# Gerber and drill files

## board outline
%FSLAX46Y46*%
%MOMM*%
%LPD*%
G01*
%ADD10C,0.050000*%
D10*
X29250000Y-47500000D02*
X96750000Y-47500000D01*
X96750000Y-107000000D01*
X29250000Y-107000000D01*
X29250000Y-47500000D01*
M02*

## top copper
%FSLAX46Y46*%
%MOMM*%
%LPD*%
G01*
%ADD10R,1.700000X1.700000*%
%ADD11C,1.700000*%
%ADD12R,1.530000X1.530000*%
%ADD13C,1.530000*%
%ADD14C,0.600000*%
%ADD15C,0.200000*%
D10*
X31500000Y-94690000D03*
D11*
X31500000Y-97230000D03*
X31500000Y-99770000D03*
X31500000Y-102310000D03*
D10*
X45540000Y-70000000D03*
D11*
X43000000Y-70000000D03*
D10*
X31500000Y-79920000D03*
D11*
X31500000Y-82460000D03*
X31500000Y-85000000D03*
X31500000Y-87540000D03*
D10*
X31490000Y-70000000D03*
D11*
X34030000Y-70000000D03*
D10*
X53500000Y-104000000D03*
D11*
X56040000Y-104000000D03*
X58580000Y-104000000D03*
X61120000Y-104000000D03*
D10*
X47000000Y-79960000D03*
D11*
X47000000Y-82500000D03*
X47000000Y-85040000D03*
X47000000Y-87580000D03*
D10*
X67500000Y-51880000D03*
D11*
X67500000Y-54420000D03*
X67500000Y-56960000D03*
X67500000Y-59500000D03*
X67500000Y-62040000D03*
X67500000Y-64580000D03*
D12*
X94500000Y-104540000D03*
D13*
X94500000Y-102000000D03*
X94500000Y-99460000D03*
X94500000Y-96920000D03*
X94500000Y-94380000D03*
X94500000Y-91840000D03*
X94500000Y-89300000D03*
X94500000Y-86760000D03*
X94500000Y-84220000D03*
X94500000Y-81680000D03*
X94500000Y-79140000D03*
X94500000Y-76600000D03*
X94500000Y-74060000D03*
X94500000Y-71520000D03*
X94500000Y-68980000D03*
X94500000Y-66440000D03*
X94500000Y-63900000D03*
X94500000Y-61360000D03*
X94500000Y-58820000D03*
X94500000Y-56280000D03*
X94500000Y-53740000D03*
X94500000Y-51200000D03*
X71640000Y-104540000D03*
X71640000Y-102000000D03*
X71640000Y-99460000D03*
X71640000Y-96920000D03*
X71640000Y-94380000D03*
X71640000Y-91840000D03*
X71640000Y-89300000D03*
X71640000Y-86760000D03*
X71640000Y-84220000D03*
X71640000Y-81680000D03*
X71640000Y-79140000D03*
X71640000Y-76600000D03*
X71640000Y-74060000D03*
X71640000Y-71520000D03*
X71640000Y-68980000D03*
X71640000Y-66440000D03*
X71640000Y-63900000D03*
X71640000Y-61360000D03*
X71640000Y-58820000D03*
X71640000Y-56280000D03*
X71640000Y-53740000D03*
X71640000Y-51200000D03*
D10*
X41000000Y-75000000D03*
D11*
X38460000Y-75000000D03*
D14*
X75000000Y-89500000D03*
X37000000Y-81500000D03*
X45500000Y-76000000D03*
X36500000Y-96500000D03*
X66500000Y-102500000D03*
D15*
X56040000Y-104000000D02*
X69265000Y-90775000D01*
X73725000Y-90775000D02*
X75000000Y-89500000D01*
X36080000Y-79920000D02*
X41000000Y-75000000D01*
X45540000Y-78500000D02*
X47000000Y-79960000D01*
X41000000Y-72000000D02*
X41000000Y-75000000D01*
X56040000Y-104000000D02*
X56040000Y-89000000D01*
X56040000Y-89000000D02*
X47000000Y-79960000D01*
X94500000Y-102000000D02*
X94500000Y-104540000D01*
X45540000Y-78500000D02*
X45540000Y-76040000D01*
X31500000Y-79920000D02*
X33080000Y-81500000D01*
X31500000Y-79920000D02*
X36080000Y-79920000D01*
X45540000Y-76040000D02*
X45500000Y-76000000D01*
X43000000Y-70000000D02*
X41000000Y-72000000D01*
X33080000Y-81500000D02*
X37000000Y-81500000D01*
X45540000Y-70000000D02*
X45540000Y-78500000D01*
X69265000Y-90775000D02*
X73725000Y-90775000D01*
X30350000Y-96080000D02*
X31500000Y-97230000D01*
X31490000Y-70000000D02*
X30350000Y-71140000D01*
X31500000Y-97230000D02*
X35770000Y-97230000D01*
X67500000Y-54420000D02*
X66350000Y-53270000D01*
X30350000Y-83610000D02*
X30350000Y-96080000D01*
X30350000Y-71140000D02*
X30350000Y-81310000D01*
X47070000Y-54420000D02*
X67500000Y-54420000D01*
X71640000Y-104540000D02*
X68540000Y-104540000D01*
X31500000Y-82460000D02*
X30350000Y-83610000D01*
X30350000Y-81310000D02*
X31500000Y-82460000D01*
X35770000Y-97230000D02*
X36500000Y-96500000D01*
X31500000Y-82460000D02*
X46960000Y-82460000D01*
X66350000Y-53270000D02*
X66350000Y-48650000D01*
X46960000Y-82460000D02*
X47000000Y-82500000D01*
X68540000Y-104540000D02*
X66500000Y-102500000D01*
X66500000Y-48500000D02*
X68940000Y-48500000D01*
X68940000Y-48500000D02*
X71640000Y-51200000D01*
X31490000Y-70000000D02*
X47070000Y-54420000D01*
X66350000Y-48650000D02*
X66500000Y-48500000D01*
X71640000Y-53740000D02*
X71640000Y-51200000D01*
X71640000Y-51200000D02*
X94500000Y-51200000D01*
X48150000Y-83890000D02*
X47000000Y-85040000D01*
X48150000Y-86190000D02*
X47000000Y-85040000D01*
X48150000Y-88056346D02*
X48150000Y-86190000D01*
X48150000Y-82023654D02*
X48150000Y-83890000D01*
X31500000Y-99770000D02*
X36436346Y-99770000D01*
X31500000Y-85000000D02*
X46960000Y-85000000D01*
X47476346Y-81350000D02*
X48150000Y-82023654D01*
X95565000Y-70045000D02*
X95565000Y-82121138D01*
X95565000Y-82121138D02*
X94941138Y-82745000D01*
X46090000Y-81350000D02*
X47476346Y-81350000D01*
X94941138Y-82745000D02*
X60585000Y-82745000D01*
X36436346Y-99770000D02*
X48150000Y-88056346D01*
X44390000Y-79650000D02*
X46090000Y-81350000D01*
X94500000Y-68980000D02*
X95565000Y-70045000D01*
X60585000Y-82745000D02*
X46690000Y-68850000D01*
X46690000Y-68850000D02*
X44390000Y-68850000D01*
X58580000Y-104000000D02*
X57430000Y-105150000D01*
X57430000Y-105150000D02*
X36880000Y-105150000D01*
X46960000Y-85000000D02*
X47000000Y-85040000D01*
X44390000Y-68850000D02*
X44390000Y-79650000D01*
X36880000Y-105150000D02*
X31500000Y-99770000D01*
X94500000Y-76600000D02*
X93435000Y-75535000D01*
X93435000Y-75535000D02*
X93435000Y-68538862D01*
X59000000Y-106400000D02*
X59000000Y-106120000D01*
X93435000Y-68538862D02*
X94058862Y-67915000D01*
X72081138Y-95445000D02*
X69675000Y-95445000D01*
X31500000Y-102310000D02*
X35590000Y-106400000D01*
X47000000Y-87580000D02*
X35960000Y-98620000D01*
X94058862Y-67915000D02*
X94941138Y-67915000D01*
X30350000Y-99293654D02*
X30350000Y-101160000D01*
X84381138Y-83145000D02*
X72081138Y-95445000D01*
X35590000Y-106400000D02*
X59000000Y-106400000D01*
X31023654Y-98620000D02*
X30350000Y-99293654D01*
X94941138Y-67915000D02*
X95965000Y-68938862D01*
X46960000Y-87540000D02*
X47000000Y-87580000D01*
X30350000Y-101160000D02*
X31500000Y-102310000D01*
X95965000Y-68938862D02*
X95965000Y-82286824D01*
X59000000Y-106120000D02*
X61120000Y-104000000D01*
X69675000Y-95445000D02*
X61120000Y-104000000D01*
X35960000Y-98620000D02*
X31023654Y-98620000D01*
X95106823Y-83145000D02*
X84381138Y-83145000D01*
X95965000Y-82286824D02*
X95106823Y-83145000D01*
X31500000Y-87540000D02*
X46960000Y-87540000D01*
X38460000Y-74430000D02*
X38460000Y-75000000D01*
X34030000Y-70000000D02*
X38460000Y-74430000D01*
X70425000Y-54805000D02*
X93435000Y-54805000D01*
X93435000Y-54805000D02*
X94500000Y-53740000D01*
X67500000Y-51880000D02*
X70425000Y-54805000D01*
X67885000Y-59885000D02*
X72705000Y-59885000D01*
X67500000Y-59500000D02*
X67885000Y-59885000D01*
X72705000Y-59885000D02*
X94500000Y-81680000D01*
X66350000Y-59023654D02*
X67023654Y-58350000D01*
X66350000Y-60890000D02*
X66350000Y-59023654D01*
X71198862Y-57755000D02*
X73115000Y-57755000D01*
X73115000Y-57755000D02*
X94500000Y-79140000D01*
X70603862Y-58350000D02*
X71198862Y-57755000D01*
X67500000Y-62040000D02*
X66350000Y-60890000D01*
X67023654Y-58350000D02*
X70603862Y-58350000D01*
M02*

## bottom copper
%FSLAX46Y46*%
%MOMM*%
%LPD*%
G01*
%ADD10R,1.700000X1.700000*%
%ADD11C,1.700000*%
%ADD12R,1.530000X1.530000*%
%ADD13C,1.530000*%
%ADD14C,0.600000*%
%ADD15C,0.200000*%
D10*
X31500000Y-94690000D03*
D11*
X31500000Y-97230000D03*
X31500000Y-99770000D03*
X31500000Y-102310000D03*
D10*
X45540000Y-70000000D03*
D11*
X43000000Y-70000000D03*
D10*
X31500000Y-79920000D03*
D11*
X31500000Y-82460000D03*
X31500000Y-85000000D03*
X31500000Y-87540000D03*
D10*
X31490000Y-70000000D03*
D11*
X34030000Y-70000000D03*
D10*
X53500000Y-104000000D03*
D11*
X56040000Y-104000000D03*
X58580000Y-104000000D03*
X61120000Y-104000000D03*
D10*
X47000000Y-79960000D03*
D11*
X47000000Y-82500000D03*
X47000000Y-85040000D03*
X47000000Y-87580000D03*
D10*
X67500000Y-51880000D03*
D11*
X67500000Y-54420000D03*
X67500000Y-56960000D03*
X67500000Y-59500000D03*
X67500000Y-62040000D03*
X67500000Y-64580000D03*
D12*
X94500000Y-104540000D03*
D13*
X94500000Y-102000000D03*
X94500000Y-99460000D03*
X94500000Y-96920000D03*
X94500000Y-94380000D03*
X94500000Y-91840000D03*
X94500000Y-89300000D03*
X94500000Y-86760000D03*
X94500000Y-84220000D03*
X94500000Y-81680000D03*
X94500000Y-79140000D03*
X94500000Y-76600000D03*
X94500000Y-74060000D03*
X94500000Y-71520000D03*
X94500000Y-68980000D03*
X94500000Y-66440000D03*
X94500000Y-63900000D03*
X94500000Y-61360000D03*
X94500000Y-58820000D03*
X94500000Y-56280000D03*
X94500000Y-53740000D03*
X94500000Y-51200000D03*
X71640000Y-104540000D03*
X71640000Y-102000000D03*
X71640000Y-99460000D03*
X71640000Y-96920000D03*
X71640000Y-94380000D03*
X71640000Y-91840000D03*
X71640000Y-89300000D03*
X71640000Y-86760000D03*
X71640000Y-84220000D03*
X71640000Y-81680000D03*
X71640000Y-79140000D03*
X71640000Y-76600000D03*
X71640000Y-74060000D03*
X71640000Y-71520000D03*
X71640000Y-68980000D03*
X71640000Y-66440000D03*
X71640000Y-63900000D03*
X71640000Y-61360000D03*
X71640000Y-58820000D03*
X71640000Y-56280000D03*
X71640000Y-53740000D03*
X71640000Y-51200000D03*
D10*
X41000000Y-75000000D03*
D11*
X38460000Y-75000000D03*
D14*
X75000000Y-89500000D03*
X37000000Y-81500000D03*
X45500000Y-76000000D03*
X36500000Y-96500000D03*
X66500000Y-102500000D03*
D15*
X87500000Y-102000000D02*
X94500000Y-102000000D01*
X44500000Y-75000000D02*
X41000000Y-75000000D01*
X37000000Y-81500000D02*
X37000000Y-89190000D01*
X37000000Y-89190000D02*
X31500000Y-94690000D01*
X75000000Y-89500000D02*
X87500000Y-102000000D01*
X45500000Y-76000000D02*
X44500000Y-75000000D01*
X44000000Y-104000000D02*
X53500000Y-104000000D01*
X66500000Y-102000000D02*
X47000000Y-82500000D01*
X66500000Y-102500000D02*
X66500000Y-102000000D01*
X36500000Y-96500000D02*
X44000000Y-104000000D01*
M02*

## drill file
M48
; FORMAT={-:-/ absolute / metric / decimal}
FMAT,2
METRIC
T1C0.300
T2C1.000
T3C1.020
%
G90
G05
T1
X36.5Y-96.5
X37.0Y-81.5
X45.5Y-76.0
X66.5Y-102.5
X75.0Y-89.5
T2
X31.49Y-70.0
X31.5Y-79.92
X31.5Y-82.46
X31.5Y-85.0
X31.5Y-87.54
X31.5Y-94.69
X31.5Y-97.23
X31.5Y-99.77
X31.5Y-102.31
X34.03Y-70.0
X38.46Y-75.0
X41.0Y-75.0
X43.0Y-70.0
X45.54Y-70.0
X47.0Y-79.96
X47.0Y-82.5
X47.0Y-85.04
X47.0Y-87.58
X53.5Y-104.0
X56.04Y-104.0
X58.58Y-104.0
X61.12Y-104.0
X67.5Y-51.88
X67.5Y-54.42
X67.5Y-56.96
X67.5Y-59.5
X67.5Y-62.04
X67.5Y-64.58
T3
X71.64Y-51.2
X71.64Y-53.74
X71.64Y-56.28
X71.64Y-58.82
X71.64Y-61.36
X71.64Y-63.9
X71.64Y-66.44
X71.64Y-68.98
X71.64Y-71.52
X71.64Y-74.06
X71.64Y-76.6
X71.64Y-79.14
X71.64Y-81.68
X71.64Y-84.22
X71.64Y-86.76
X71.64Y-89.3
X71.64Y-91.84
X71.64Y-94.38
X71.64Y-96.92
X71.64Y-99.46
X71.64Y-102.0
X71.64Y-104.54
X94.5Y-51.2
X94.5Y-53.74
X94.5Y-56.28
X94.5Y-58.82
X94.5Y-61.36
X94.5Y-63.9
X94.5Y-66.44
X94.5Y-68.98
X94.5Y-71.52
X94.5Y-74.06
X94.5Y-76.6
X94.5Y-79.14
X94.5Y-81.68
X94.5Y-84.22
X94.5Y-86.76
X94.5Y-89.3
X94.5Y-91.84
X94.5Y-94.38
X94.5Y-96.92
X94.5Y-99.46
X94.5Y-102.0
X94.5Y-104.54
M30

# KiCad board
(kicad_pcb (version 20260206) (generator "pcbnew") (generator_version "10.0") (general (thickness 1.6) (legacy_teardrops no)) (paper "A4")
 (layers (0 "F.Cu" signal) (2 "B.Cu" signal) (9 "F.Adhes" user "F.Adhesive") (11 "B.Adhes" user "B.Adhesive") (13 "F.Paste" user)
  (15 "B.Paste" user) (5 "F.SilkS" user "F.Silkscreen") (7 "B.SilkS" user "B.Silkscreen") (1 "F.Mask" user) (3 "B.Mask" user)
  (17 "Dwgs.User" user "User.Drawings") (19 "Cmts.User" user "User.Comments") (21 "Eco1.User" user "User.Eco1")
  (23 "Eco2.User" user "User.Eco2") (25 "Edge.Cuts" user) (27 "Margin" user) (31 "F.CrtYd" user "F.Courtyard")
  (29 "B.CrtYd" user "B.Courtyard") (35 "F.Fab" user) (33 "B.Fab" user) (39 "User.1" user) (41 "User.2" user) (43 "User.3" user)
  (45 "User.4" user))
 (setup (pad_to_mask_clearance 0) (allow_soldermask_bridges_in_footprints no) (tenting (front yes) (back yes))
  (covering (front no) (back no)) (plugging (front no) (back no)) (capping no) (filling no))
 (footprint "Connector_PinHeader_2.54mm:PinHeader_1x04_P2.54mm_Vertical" (layer "F.Cu") (at 31.5 94.69)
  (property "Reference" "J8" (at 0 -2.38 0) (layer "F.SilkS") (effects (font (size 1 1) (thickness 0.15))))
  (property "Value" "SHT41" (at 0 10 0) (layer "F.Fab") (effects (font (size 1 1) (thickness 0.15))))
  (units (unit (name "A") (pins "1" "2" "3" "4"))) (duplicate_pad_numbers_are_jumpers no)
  (pad "1" thru_hole rect (at 0 0) (size 1.7 1.7) (drill 1) (layers "*.Cu" "*.Mask") (remove_unused_layers no) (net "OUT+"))
  (pad "2" thru_hole circle (at 0 2.54) (size 1.7 1.7) (drill 1) (layers "*.Cu" "*.Mask") (remove_unused_layers no) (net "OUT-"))
  (pad "3" thru_hole circle (at 0 5.08) (size 1.7 1.7) (drill 1) (layers "*.Cu" "*.Mask") (remove_unused_layers no) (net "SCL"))
  (pad "4" thru_hole circle (at 0 7.62) (size 1.7 1.7) (drill 1) (layers "*.Cu" "*.Mask") (remove_unused_layers no) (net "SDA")))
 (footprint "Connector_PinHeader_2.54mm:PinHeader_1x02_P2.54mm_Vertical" (layer "F.Cu") (at 45.54 70 -90)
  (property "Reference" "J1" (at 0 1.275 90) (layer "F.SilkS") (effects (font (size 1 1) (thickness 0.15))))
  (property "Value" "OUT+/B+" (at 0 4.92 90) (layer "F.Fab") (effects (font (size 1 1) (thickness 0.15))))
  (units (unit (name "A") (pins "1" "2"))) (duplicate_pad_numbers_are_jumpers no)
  (pad "1" thru_hole rect (at 0 0 270) (size 1.7 1.7) (drill 1) (layers "*.Cu" "*.Mask") (remove_unused_layers no) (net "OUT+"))
  (pad "2" thru_hole circle (at 0 2.54 270) (size 1.7 1.7) (drill 1) (layers "*.Cu" "*.Mask") (remove_unused_layers no) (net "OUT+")))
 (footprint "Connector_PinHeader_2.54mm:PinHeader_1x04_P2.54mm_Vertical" (layer "F.Cu") (at 31.5 79.92)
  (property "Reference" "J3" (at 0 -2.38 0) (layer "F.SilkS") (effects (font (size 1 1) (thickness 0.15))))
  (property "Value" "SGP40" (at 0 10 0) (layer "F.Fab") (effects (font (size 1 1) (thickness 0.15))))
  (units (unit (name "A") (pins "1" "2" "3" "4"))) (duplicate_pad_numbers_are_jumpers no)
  (pad "1" thru_hole rect (at 0 0) (size 1.7 1.7) (drill 1) (layers "*.Cu" "*.Mask") (remove_unused_layers no) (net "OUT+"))
  (pad "2" thru_hole circle (at 0 2.54) (size 1.7 1.7) (drill 1) (layers "*.Cu" "*.Mask") (remove_unused_layers no) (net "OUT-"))
  (pad "3" thru_hole circle (at 0 5.08) (size 1.7 1.7) (drill 1) (layers "*.Cu" "*.Mask") (remove_unused_layers no) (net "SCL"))
  (pad "4" thru_hole circle (at 0 7.62) (size 1.7 1.7) (drill 1) (layers "*.Cu" "*.Mask") (remove_unused_layers no) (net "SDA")))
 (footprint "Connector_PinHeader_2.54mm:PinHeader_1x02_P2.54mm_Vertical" (layer "F.Cu") (at 31.49 70 90)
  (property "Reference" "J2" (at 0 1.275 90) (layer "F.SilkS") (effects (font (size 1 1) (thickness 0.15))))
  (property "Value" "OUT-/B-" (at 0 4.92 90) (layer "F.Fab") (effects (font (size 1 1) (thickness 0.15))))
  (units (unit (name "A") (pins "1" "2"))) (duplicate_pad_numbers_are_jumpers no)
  (pad "1" thru_hole rect (at 0 0 90) (size 1.7 1.7) (drill 1) (layers "*.Cu" "*.Mask") (remove_unused_layers no) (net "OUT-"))
  (pad "2" thru_hole circle (at 0 2.54 90) (size 1.7 1.7) (drill 1) (layers "*.Cu" "*.Mask") (remove_unused_layers no)
   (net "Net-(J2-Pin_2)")))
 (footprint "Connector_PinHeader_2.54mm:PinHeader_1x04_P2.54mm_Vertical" (layer "F.Cu") (at 53.5 104 90)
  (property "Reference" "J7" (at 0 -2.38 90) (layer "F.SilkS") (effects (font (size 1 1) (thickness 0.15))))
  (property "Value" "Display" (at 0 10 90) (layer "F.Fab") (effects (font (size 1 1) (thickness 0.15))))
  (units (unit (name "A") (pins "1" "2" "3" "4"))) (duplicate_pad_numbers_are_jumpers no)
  (pad "1" thru_hole rect (at 0 0 90) (size 1.7 1.7) (drill 1) (layers "*.Cu" "*.Mask") (remove_unused_layers no) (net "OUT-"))
  (pad "2" thru_hole circle (at 0 2.54 90) (size 1.7 1.7) (drill 1) (layers "*.Cu" "*.Mask") (remove_unused_layers no) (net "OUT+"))
  (pad "3" thru_hole circle (at 0 5.08 90) (size 1.7 1.7) (drill 1) (layers "*.Cu" "*.Mask") (remove_unused_layers no) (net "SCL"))
  (pad "4" thru_hole circle (at 0 7.62 90) (size 1.7 1.7) (drill 1) (layers "*.Cu" "*.Mask") (remove_unused_layers no) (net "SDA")))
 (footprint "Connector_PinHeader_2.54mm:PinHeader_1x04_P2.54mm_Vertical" (layer "F.Cu") (at 47 79.96)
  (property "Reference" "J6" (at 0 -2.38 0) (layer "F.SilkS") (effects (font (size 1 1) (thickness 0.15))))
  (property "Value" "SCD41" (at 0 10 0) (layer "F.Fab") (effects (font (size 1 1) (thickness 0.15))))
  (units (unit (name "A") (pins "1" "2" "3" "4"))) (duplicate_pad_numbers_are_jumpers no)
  (pad "1" thru_hole rect (at 0 0) (size 1.7 1.7) (drill 1) (layers "*.Cu" "*.Mask") (remove_unused_layers no) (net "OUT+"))
  (pad "2" thru_hole circle (at 0 2.54) (size 1.7 1.7) (drill 1) (layers "*.Cu" "*.Mask") (remove_unused_layers no) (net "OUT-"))
  (pad "3" thru_hole circle (at 0 5.08) (size 1.7 1.7) (drill 1) (layers "*.Cu" "*.Mask") (remove_unused_layers no) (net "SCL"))
  (pad "4" thru_hole circle (at 0 7.62) (size 1.7 1.7) (drill 1) (layers "*.Cu" "*.Mask") (remove_unused_layers no) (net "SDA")))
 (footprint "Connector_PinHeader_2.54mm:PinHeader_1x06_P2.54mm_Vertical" (layer "F.Cu") (at 67.5 51.88)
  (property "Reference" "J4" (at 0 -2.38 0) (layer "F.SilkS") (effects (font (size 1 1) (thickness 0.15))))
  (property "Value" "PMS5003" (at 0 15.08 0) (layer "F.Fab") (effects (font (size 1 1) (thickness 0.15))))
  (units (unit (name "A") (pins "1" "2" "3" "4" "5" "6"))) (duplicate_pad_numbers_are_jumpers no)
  (pad "1" thru_hole rect (at 0 0) (size 1.7 1.7) (drill 1) (layers "*.Cu" "*.Mask") (remove_unused_layers no) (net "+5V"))
  (pad "2" thru_hole circle (at 0 2.54) (size 1.7 1.7) (drill 1) (layers "*.Cu" "*.Mask") (remove_unused_layers no) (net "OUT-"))
  (pad "3" thru_hole circle (at 0 5.08) (size 1.7 1.7) (drill 1) (layers "*.Cu" "*.Mask") (remove_unused_layers no)
   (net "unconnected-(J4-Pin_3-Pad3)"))
  (pad "4" thru_hole circle (at 0 7.62) (size 1.7 1.7) (drill 1) (layers "*.Cu" "*.Mask") (remove_unused_layers no) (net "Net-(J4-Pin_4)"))
  (pad "5" thru_hole circle (at 0 10.16) (size 1.7 1.7) (drill 1) (layers "*.Cu" "*.Mask") (remove_unused_layers no) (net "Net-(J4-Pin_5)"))
  (pad "6" thru_hole circle (at 0 12.7) (size 1.7 1.7) (drill 1) (layers "*.Cu" "*.Mask") (remove_unused_layers no)
   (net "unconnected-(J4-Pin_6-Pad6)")))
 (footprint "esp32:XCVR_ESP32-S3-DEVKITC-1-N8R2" (layer "F.Cu") (at 83.07 74.57 180)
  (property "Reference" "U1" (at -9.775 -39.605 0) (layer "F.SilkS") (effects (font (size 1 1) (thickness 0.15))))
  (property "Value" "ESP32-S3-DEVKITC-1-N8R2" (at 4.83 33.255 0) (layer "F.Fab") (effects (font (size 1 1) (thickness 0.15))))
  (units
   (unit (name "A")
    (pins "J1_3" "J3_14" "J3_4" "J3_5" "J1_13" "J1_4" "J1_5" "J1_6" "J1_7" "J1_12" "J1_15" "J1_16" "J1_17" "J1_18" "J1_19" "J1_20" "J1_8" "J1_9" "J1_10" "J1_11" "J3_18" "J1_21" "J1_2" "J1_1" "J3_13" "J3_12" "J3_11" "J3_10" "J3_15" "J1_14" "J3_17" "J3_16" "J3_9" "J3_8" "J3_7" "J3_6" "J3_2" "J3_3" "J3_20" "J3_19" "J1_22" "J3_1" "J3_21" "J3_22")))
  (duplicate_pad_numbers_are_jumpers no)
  (pad "J1_1" thru_hole rect (at -11.43 -29.97 180) (size 1.53 1.53) (drill 1.02) (layers "*.Cu" "*.Mask") (remove_unused_layers no)
   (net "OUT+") (solder_mask_margin 0.102))
  (pad "J1_2" thru_hole circle (at -11.43 -27.43 180) (size 1.53 1.53) (drill 1.02) (layers "*.Cu" "*.Mask") (remove_unused_layers no)
   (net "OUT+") (solder_mask_margin 0.102))
  (pad "J1_3" thru_hole circle (at -11.43 -24.89 180) (size 1.53 1.53) (drill 1.02) (layers "*.Cu" "*.Mask") (remove_unused_layers no)
   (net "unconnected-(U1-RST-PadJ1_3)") (solder_mask_margin 0.102))
  (pad "J1_4" thru_hole circle (at -11.43 -22.35 180) (size 1.53 1.53) (drill 1.02) (layers "*.Cu" "*.Mask") (remove_unused_layers no)
   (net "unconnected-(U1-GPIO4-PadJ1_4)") (solder_mask_margin 0.102))
  (pad "J1_5" thru_hole circle (at -11.43 -19.81 180) (size 1.53 1.53) (drill 1.02) (layers "*.Cu" "*.Mask") (remove_unused_layers no)
   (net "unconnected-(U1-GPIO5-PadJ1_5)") (solder_mask_margin 0.102))
  (pad "J1_6" thru_hole circle (at -11.43 -17.27 180) (size 1.53 1.53) (drill 1.02) (layers "*.Cu" "*.Mask") (remove_unused_layers no)
   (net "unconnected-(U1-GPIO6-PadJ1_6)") (solder_mask_margin 0.102))
  (pad "J1_7" thru_hole circle (at -11.43 -14.73 180) (size 1.53 1.53) (drill 1.02) (layers "*.Cu" "*.Mask") (remove_unused_layers no)
   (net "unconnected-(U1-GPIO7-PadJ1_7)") (solder_mask_margin 0.102))
  (pad "J1_8" thru_hole circle (at -11.43 -12.19 180) (size 1.53 1.53) (drill 1.02) (layers "*.Cu" "*.Mask") (remove_unused_layers no)
   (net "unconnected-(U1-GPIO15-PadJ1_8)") (solder_mask_margin 0.102))
  (pad "J1_9" thru_hole circle (at -11.43 -9.65 180) (size 1.53 1.53) (drill 1.02) (layers "*.Cu" "*.Mask") (remove_unused_layers no)
   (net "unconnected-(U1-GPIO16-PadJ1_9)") (solder_mask_margin 0.102))
  (pad "J1_10" thru_hole circle (at -11.43 -7.11 180) (size 1.53 1.53) (drill 1.02) (layers "*.Cu" "*.Mask") (remove_unused_layers no)
   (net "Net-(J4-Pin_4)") (solder_mask_margin 0.102))
  (pad "J1_11" thru_hole circle (at -11.43 -4.57 180) (size 1.53 1.53) (drill 1.02) (layers "*.Cu" "*.Mask") (remove_unused_layers no)
   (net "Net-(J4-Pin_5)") (solder_mask_margin 0.102))
  (pad "J1_12" thru_hole circle (at -11.43 -2.03 180) (size 1.53 1.53) (drill 1.02) (layers "*.Cu" "*.Mask") (remove_unused_layers no)
   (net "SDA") (solder_mask_margin 0.102))
  (pad "J1_13" thru_hole circle (at -11.43 0.51 180) (size 1.53 1.53) (drill 1.02) (layers "*.Cu" "*.Mask") (remove_unused_layers no)
   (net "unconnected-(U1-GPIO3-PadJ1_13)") (solder_mask_margin 0.102))
  (pad "J1_14" thru_hole circle (at -11.43 3.05 180) (size 1.53 1.53) (drill 1.02) (layers "*.Cu" "*.Mask") (remove_unused_layers no)
   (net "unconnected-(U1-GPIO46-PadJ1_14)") (solder_mask_margin 0.102))
  (pad "J1_15" thru_hole circle (at -11.43 5.59 180) (size 1.53 1.53) (drill 1.02) (layers "*.Cu" "*.Mask") (remove_unused_layers no)
   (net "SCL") (solder_mask_margin 0.102))
  (pad "J1_16" thru_hole circle (at -11.43 8.13 180) (size 1.53 1.53) (drill 1.02) (layers "*.Cu" "*.Mask") (remove_unused_layers no)
   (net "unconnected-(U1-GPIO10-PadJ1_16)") (solder_mask_margin 0.102))
  (pad "J1_17" thru_hole circle (at -11.43 10.67 180) (size 1.53 1.53) (drill 1.02) (layers "*.Cu" "*.Mask") (remove_unused_layers no)
   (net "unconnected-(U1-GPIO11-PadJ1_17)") (solder_mask_margin 0.102))
  (pad "J1_18" thru_hole circle (at -11.43 13.21 180) (size 1.53 1.53) (drill 1.02) (layers "*.Cu" "*.Mask") (remove_unused_layers no)
   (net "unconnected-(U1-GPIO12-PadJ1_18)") (solder_mask_margin 0.102))
  (pad "J1_19" thru_hole circle (at -11.43 15.75 180) (size 1.53 1.53) (drill 1.02) (layers "*.Cu" "*.Mask") (remove_unused_layers no)
   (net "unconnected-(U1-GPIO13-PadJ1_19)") (solder_mask_margin 0.102))
  (pad "J1_20" thru_hole circle (at -11.43 18.29 180) (size 1.53 1.53) (drill 1.02) (layers "*.Cu" "*.Mask") (remove_unused_layers no)
   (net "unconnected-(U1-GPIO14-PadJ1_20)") (solder_mask_margin 0.102))
  (pad "J1_21" thru_hole circle (at -11.43 20.83 180) (size 1.53 1.53) (drill 1.02) (layers "*.Cu" "*.Mask") (remove_unused_layers no)
   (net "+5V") (solder_mask_margin 0.102))
  (pad "J1_22" thru_hole circle (at -11.43 23.37 180) (size 1.53 1.53) (drill 1.02) (layers "*.Cu" "*.Mask") (remove_unused_layers no)
   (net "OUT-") (solder_mask_margin 0.102))
  (pad "J3_1" thru_hole circle (at 11.43 -29.97 180) (size 1.53 1.53) (drill 1.02) (layers "*.Cu" "*.Mask") (remove_unused_layers no)
   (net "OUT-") (solder_mask_margin 0.102))
  (pad "J3_2" thru_hole circle (at 11.43 -27.43 180) (size 1.53 1.53) (drill 1.02) (layers "*.Cu" "*.Mask") (remove_unused_layers no)
   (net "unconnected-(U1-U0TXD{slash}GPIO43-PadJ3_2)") (solder_mask_margin 0.102))
  (pad "J3_3" thru_hole circle (at 11.43 -24.89 180) (size 1.53 1.53) (drill 1.02) (layers "*.Cu" "*.Mask") (remove_unused_layers no)
   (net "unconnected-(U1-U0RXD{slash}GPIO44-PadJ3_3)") (solder_mask_margin 0.102))
  (pad "J3_4" thru_hole circle (at 11.43 -22.35 180) (size 1.53 1.53) (drill 1.02) (layers "*.Cu" "*.Mask") (remove_unused_layers no)
   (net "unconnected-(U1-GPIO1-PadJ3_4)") (solder_mask_margin 0.102))
  (pad "J3_5" thru_hole circle (at 11.43 -19.81 180) (size 1.53 1.53) (drill 1.02) (layers "*.Cu" "*.Mask") (remove_unused_layers no)
   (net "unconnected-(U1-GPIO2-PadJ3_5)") (solder_mask_margin 0.102))
  (pad "J3_6" thru_hole circle (at 11.43 -17.27 180) (size 1.53 1.53) (drill 1.02) (layers "*.Cu" "*.Mask") (remove_unused_layers no)
   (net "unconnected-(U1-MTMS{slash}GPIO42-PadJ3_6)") (solder_mask_margin 0.102))
  (pad "J3_7" thru_hole circle (at 11.43 -14.73 180) (size 1.53 1.53) (drill 1.02) (layers "*.Cu" "*.Mask") (remove_unused_layers no)
   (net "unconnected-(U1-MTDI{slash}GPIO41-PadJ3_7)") (solder_mask_margin 0.102))
  (pad "J3_8" thru_hole circle (at 11.43 -12.19 180) (size 1.53 1.53) (drill 1.02) (layers "*.Cu" "*.Mask") (remove_unused_layers no)
   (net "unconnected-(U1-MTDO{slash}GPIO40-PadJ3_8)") (solder_mask_margin 0.102))
  (pad "J3_9" thru_hole circle (at 11.43 -9.65 180) (size 1.53 1.53) (drill 1.02) (layers "*.Cu" "*.Mask") (remove_unused_layers no)
   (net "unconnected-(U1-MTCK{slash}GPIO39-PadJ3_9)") (solder_mask_margin 0.102))
  (pad "J3_10" thru_hole circle (at 11.43 -7.11 180) (size 1.53 1.53) (drill 1.02) (layers "*.Cu" "*.Mask") (remove_unused_layers no)
   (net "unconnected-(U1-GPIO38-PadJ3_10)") (solder_mask_margin 0.102))
  (pad "J3_11" thru_hole circle (at 11.43 -4.57 180) (size 1.53 1.53) (drill 1.02) (layers "*.Cu" "*.Mask") (remove_unused_layers no)
   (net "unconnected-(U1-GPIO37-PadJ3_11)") (solder_mask_margin 0.102))
  (pad "J3_12" thru_hole circle (at 11.43 -2.03 180) (size 1.53 1.53) (drill 1.02) (layers "*.Cu" "*.Mask") (remove_unused_layers no)
   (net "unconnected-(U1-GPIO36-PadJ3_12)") (solder_mask_margin 0.102))
  (pad "J3_13" thru_hole circle (at 11.43 0.51 180) (size 1.53 1.53) (drill 1.02) (layers "*.Cu" "*.Mask") (remove_unused_layers no)
   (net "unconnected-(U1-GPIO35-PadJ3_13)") (solder_mask_margin 0.102))
  (pad "J3_14" thru_hole circle (at 11.43 3.05 180) (size 1.53 1.53) (drill 1.02) (layers "*.Cu" "*.Mask") (remove_unused_layers no)
   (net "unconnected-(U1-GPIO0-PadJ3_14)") (solder_mask_margin 0.102))
  (pad "J3_15" thru_hole circle (at 11.43 5.59 180) (size 1.53 1.53) (drill 1.02) (layers "*.Cu" "*.Mask") (remove_unused_layers no)
   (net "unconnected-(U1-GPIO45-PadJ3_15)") (solder_mask_margin 0.102))
  (pad "J3_16" thru_hole circle (at 11.43 8.13 180) (size 1.53 1.53) (drill 1.02) (layers "*.Cu" "*.Mask") (remove_unused_layers no)
   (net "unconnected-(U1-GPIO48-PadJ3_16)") (solder_mask_margin 0.102))
  (pad "J3_17" thru_hole circle (at 11.43 10.67 180) (size 1.53 1.53) (drill 1.02) (layers "*.Cu" "*.Mask") (remove_unused_layers no)
   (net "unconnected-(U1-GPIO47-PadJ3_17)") (solder_mask_margin 0.102))
  (pad "J3_18" thru_hole circle (at 11.43 13.21 180) (size 1.53 1.53) (drill 1.02) (layers "*.Cu" "*.Mask") (remove_unused_layers no)
   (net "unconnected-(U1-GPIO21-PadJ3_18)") (solder_mask_margin 0.102))
  (pad "J3_19" thru_hole circle (at 11.43 15.75 180) (size 1.53 1.53) (drill 1.02) (layers "*.Cu" "*.Mask") (remove_unused_layers no)
   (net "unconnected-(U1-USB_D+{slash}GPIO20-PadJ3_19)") (solder_mask_margin 0.102))
  (pad "J3_20" thru_hole circle (at 11.43 18.29 180) (size 1.53 1.53) (drill 1.02) (layers "*.Cu" "*.Mask") (remove_unused_layers no)
   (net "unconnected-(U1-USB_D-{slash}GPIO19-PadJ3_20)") (solder_mask_margin 0.102))
  (pad "J3_21" thru_hole circle (at 11.43 20.83 180) (size 1.53 1.53) (drill 1.02) (layers "*.Cu" "*.Mask") (remove_unused_layers no)
   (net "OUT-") (solder_mask_margin 0.102))
  (pad "J3_22" thru_hole circle (at 11.43 23.37 180) (size 1.53 1.53) (drill 1.02) (layers "*.Cu" "*.Mask") (remove_unused_layers no)
   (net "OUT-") (solder_mask_margin 0.102)))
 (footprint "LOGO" (layer "F.Cu") (at 63 98)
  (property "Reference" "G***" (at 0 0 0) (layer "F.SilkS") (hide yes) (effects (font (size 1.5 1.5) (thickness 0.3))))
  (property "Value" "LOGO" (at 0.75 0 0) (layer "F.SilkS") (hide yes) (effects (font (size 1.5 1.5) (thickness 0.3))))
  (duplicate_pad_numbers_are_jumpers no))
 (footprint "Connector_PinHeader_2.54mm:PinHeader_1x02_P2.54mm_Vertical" (layer "F.Cu") (at 41 75 -90)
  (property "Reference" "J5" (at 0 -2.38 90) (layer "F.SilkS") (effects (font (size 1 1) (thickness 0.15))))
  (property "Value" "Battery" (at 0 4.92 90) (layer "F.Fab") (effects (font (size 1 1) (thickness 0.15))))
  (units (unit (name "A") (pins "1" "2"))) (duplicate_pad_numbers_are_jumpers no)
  (pad "1" thru_hole rect (at 0 0 270) (size 1.7 1.7) (drill 1) (layers "*.Cu" "*.Mask") (remove_unused_layers no) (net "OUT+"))
  (pad "2" thru_hole circle (at 0 2.54 270) (size 1.7 1.7) (drill 1) (layers "*.Cu" "*.Mask") (remove_unused_layers no)
   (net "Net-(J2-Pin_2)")))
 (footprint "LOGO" (layer "F.Cu") (at 49.5 98)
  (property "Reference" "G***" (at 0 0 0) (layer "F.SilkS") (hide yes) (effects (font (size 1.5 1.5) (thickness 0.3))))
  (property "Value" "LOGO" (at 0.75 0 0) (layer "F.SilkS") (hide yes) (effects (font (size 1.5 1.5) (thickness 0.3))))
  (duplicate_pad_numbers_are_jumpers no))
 (gr_rect (start 29.25 47.5) (end 96.75 107) (stroke (width 0.05) (type default)) (fill no) (layer "Edge.Cuts"))
 (segment (start 56.04 104) (end 69.265 90.775) (width 0.2) (layer "F.Cu") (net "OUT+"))
 (segment (start 73.725 90.775) (end 75 89.5) (width 0.2) (layer "F.Cu") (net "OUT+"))
 (segment (start 36.08 79.92) (end 41 75) (width 0.2) (layer "F.Cu") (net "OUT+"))
 (segment (start 45.54 78.5) (end 47 79.96) (width 0.2) (layer "F.Cu") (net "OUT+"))
 (segment (start 41 72) (end 41 75) (width 0.2) (layer "F.Cu") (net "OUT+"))
 (segment (start 56.04 104) (end 56.04 89) (width 0.2) (layer "F.Cu") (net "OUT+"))
 (segment (start 56.04 89) (end 47 79.96) (width 0.2) (layer "F.Cu") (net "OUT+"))
 (segment (start 94.5 102) (end 94.5 104.54) (width 0.2) (layer "F.Cu") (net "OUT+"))
 (segment (start 45.54 78.5) (end 45.54 76.04) (width 0.2) (layer "F.Cu") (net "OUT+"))
 (segment (start 31.5 79.92) (end 33.08 81.5) (width 0.2) (layer "F.Cu") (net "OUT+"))
 (segment (start 31.5 79.92) (end 36.08 79.92) (width 0.2) (layer "F.Cu") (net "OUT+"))
 (segment (start 45.54 76.04) (end 45.5 76) (width 0.2) (layer "F.Cu") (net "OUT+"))
 (segment (start 43 70) (end 41 72) (width 0.2) (layer "F.Cu") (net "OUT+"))
 (segment (start 33.08 81.5) (end 37 81.5) (width 0.2) (layer "F.Cu") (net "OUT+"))
 (segment (start 45.54 70) (end 45.54 78.5) (width 0.2) (layer "F.Cu") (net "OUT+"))
 (segment (start 69.265 90.775) (end 73.725 90.775) (width 0.2) (layer "F.Cu") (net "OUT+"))
 (via (at 75 89.5) (size 0.6) (drill 0.3) (layers "F.Cu" "B.Cu") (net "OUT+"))
 (via (at 37 81.5) (size 0.6) (drill 0.3) (layers "F.Cu" "B.Cu") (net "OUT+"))
 (via (at 45.5 76) (size 0.6) (drill 0.3) (layers "F.Cu" "B.Cu") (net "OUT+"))
 (segment (start 87.5 102) (end 94.5 102) (width 0.2) (layer "B.Cu") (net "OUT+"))
 (segment (start 44.5 75) (end 41 75) (width 0.2) (layer "B.Cu") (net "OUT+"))
 (segment (start 37 81.5) (end 37 89.19) (width 0.2) (layer "B.Cu") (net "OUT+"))
 (segment (start 37 89.19) (end 31.5 94.69) (width 0.2) (layer "B.Cu") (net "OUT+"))
 (segment (start 75 89.5) (end 87.5 102) (width 0.2) (layer "B.Cu") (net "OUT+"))
 (segment (start 45.5 76) (end 44.5 75) (width 0.2) (layer "B.Cu") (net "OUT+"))
 (segment (start 30.35 96.08) (end 31.5 97.23) (width 0.2) (layer "F.Cu") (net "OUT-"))
 (segment (start 31.49 70) (end 30.35 71.14) (width 0.2) (layer "F.Cu") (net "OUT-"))
 (segment (start 31.5 97.23) (end 35.77 97.23) (width 0.2) (layer "F.Cu") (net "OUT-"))
 (segment (start 67.5 54.42) (end 66.35 53.27) (width 0.2) (layer "F.Cu") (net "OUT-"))
 (segment (start 30.35 83.61) (end 30.35 96.08) (width 0.2) (layer "F.Cu") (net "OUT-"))
 (segment (start 30.35 71.14) (end 30.35 81.31) (width 0.2) (layer "F.Cu") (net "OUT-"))
 (segment (start 47.07 54.42) (end 67.5 54.42) (width 0.2) (layer "F.Cu") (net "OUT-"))
 (segment (start 71.64 104.54) (end 68.54 104.54) (width 0.2) (layer "F.Cu") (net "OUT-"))
 (segment (start 31.5 82.46) (end 30.35 83.61) (width 0.2) (layer "F.Cu") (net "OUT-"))
 (segment (start 30.35 81.31) (end 31.5 82.46) (width 0.2) (layer "F.Cu") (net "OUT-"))
 (segment (start 35.77 97.23) (end 36.5 96.5) (width 0.2) (layer "F.Cu") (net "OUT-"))
 (segment (start 31.5 82.46) (end 46.96 82.46) (width 0.2) (layer "F.Cu") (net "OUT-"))
 (segment (start 66.35 53.27) (end 66.35 48.65) (width 0.2) (layer "F.Cu") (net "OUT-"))
 (segment (start 46.96 82.46) (end 47 82.5) (width 0.2) (layer "F.Cu") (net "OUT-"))
 (segment (start 68.54 104.54) (end 66.5 102.5) (width 0.2) (layer "F.Cu") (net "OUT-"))
 (segment (start 66.5 48.5) (end 68.94 48.5) (width 0.2) (layer "F.Cu") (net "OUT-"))
 (segment (start 68.94 48.5) (end 71.64 51.2) (width 0.2) (layer "F.Cu") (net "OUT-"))
 (segment (start 31.49 70) (end 47.07 54.42) (width 0.2) (layer "F.Cu") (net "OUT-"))
 (segment (start 66.35 48.65) (end 66.5 48.5) (width 0.2) (layer "F.Cu") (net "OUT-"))
 (segment (start 71.64 53.74) (end 71.64 51.2) (width 0.2) (layer "F.Cu") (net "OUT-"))
 (segment (start 71.64 51.2) (end 94.5 51.2) (width 0.2) (layer "F.Cu") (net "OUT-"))
 (via (at 36.5 96.5) (size 0.6) (drill 0.3) (layers "F.Cu" "B.Cu") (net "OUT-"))
 (via (at 66.5 102.5) (size 0.6) (drill 0.3) (layers "F.Cu" "B.Cu") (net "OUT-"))
 (segment (start 44 104) (end 53.5 104) (width 0.2) (layer "B.Cu") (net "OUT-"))
 (segment (start 66.5 102) (end 47 82.5) (width 0.2) (layer "B.Cu") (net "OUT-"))
 (segment (start 66.5 102.5) (end 66.5 102) (width 0.2) (layer "B.Cu") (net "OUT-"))
 (segment (start 36.5 96.5) (end 44 104) (width 0.2) (layer "B.Cu") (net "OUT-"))
 (segment (start 48.15 83.89) (end 47 85.04) (width 0.2) (layer "F.Cu") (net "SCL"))
 (segment (start 48.15 86.19) (end 47 85.04) (width 0.2) (layer "F.Cu") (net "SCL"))
 (segment (start 48.15 88.056346) (end 48.15 86.19) (width 0.2) (layer "F.Cu") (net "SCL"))
 (segment (start 48.15 82.023654) (end 48.15 83.89) (width 0.2) (layer "F.Cu") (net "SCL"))
 (segment (start 31.5 99.77) (end 36.436346 99.77) (width 0.2) (layer "F.Cu") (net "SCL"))
 (segment (start 31.5 85) (end 46.96 85) (width 0.2) (layer "F.Cu") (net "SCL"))
 (segment (start 47.476346 81.35) (end 48.15 82.023654) (width 0.2) (layer "F.Cu") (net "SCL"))
 (segment (start 95.565 70.045) (end 95.565 82.121138) (width 0.2) (layer "F.Cu") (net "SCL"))
 (segment (start 95.565 82.121138) (end 94.941138 82.745) (width 0.2) (layer "F.Cu") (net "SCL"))
 (segment (start 46.09 81.35) (end 47.476346 81.35) (width 0.2) (layer "F.Cu") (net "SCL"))
 (segment (start 94.941138 82.745) (end 60.585 82.745) (width 0.2) (layer "F.Cu") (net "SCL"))
 (segment (start 36.436346 99.77) (end 48.15 88.056346) (width 0.2) (layer "F.Cu") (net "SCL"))
 (segment (start 44.39 79.65) (end 46.09 81.35) (width 0.2) (layer "F.Cu") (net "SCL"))
 (segment (start 94.5 68.98) (end 95.565 70.045) (width 0.2) (layer "F.Cu") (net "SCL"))
 (segment (start 60.585 82.745) (end 46.69 68.85) (width 0.2) (layer "F.Cu") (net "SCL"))
 (segment (start 46.69 68.85) (end 44.39 68.85) (width 0.2) (layer "F.Cu") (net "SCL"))
 (segment (start 58.58 104) (end 57.43 105.15) (width 0.2) (layer "F.Cu") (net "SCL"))
 (segment (start 57.43 105.15) (end 36.88 105.15) (width 0.2) (layer "F.Cu") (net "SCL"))
 (segment (start 46.96 85) (end 47 85.04) (width 0.2) (layer "F.Cu") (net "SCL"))
 (segment (start 44.39 68.85) (end 44.39 79.65) (width 0.2) (layer "F.Cu") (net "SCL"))
 (segment (start 36.88 105.15) (end 31.5 99.77) (width 0.2) (layer "F.Cu") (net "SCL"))
 (segment (start 94.5 76.6) (end 93.435 75.535) (width 0.2) (layer "F.Cu") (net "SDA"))
 (segment (start 93.435 75.535) (end 93.435 68.538862) (width 0.2) (layer "F.Cu") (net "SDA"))
 (segment (start 59 106.4) (end 59 106.12) (width 0.2) (layer "F.Cu") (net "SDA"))
 (segment (start 93.435 68.538862) (end 94.058862 67.915) (width 0.2) (layer "F.Cu") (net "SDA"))
 (segment (start 72.081138 95.445) (end 69.675 95.445) (width 0.2) (layer "F.Cu") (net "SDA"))
 (segment (start 31.5 102.31) (end 35.59 106.4) (width 0.2) (layer "F.Cu") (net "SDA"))
 (segment (start 47 87.58) (end 35.96 98.62) (width 0.2) (layer "F.Cu") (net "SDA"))
 (segment (start 94.058862 67.915) (end 94.941138 67.915) (width 0.2) (layer "F.Cu") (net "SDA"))
 (segment (start 30.35 99.293654) (end 30.35 101.16) (width 0.2) (layer "F.Cu") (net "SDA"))
 (segment (start 84.381138 83.145) (end 72.081138 95.445) (width 0.2) (layer "F.Cu") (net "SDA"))
 (segment (start 35.59 106.4) (end 59 106.4) (width 0.2) (layer "F.Cu") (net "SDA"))
 (segment (start 31.023654 98.62) (end 30.35 99.293654) (width 0.2) (layer "F.Cu") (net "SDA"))
 (segment (start 94.941138 67.915) (end 95.965 68.938862) (width 0.2) (layer "F.Cu") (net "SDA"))
 (segment (start 46.96 87.54) (end 47 87.58) (width 0.2) (layer "F.Cu") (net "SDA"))
 (segment (start 30.35 101.16) (end 31.5 102.31) (width 0.2) (layer "F.Cu") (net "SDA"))
 (segment (start 95.965 68.938862) (end 95.965 82.286824) (width 0.2) (layer "F.Cu") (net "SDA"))
 (segment (start 59 106.12) (end 61.12 104) (width 0.2) (layer "F.Cu") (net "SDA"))
 (segment (start 69.675 95.445) (end 61.12 104) (width 0.2) (layer "F.Cu") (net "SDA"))
 (segment (start 35.96 98.62) (end 31.023654 98.62) (width 0.2) (layer "F.Cu") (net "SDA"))
 (segment (start 95.106823 83.145) (end 84.381138 83.145) (width 0.2) (layer "F.Cu") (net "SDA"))
 (segment (start 95.965 82.286824) (end 95.106823 83.145) (width 0.2) (layer "F.Cu") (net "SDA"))
 (segment (start 31.5 87.54) (end 46.96 87.54) (width 0.2) (layer "F.Cu") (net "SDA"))
 (segment (start 38.46 74.43) (end 38.46 75) (width 0.2) (layer "F.Cu") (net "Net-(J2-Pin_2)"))
 (segment (start 34.03 70) (end 38.46 74.43) (width 0.2) (layer "F.Cu") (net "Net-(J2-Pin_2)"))
 (segment (start 70.425 54.805) (end 93.435 54.805) (width 0.2) (layer "F.Cu") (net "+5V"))
 (segment (start 93.435 54.805) (end 94.5 53.74) (width 0.2) (layer "F.Cu") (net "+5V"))
 (segment (start 67.5 51.88) (end 70.425 54.805) (width 0.2) (layer "F.Cu") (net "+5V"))
 (segment (start 67.885 59.885) (end 72.705 59.885) (width 0.2) (layer "F.Cu") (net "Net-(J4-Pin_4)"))
 (segment (start 67.5 59.5) (end 67.885 59.885) (width 0.2) (layer "F.Cu") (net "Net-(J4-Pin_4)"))
 (segment (start 72.705 59.885) (end 94.5 81.68) (width 0.2) (layer "F.Cu") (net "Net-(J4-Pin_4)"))
 (segment (start 66.35 59.023654) (end 67.023654 58.35) (width 0.2) (layer "F.Cu") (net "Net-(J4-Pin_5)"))
 (segment (start 66.35 60.89) (end 66.35 59.023654) (width 0.2) (layer "F.Cu") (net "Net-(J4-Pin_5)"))
 (segment (start 71.198862 57.755) (end 73.115 57.755) (width 0.2) (layer "F.Cu") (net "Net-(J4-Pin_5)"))
 (segment (start 73.115 57.755) (end 94.5 79.14) (width 0.2) (layer "F.Cu") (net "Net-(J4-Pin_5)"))
 (segment (start 70.603862 58.35) (end 71.198862 57.755) (width 0.2) (layer "F.Cu") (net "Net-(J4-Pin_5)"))
 (segment (start 67.5 62.04) (end 66.35 60.89) (width 0.2) (layer "F.Cu") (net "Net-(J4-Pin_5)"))
 (segment (start 67.023654 58.35) (end 70.603862 58.35) (width 0.2) (layer "F.Cu") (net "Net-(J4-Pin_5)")))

